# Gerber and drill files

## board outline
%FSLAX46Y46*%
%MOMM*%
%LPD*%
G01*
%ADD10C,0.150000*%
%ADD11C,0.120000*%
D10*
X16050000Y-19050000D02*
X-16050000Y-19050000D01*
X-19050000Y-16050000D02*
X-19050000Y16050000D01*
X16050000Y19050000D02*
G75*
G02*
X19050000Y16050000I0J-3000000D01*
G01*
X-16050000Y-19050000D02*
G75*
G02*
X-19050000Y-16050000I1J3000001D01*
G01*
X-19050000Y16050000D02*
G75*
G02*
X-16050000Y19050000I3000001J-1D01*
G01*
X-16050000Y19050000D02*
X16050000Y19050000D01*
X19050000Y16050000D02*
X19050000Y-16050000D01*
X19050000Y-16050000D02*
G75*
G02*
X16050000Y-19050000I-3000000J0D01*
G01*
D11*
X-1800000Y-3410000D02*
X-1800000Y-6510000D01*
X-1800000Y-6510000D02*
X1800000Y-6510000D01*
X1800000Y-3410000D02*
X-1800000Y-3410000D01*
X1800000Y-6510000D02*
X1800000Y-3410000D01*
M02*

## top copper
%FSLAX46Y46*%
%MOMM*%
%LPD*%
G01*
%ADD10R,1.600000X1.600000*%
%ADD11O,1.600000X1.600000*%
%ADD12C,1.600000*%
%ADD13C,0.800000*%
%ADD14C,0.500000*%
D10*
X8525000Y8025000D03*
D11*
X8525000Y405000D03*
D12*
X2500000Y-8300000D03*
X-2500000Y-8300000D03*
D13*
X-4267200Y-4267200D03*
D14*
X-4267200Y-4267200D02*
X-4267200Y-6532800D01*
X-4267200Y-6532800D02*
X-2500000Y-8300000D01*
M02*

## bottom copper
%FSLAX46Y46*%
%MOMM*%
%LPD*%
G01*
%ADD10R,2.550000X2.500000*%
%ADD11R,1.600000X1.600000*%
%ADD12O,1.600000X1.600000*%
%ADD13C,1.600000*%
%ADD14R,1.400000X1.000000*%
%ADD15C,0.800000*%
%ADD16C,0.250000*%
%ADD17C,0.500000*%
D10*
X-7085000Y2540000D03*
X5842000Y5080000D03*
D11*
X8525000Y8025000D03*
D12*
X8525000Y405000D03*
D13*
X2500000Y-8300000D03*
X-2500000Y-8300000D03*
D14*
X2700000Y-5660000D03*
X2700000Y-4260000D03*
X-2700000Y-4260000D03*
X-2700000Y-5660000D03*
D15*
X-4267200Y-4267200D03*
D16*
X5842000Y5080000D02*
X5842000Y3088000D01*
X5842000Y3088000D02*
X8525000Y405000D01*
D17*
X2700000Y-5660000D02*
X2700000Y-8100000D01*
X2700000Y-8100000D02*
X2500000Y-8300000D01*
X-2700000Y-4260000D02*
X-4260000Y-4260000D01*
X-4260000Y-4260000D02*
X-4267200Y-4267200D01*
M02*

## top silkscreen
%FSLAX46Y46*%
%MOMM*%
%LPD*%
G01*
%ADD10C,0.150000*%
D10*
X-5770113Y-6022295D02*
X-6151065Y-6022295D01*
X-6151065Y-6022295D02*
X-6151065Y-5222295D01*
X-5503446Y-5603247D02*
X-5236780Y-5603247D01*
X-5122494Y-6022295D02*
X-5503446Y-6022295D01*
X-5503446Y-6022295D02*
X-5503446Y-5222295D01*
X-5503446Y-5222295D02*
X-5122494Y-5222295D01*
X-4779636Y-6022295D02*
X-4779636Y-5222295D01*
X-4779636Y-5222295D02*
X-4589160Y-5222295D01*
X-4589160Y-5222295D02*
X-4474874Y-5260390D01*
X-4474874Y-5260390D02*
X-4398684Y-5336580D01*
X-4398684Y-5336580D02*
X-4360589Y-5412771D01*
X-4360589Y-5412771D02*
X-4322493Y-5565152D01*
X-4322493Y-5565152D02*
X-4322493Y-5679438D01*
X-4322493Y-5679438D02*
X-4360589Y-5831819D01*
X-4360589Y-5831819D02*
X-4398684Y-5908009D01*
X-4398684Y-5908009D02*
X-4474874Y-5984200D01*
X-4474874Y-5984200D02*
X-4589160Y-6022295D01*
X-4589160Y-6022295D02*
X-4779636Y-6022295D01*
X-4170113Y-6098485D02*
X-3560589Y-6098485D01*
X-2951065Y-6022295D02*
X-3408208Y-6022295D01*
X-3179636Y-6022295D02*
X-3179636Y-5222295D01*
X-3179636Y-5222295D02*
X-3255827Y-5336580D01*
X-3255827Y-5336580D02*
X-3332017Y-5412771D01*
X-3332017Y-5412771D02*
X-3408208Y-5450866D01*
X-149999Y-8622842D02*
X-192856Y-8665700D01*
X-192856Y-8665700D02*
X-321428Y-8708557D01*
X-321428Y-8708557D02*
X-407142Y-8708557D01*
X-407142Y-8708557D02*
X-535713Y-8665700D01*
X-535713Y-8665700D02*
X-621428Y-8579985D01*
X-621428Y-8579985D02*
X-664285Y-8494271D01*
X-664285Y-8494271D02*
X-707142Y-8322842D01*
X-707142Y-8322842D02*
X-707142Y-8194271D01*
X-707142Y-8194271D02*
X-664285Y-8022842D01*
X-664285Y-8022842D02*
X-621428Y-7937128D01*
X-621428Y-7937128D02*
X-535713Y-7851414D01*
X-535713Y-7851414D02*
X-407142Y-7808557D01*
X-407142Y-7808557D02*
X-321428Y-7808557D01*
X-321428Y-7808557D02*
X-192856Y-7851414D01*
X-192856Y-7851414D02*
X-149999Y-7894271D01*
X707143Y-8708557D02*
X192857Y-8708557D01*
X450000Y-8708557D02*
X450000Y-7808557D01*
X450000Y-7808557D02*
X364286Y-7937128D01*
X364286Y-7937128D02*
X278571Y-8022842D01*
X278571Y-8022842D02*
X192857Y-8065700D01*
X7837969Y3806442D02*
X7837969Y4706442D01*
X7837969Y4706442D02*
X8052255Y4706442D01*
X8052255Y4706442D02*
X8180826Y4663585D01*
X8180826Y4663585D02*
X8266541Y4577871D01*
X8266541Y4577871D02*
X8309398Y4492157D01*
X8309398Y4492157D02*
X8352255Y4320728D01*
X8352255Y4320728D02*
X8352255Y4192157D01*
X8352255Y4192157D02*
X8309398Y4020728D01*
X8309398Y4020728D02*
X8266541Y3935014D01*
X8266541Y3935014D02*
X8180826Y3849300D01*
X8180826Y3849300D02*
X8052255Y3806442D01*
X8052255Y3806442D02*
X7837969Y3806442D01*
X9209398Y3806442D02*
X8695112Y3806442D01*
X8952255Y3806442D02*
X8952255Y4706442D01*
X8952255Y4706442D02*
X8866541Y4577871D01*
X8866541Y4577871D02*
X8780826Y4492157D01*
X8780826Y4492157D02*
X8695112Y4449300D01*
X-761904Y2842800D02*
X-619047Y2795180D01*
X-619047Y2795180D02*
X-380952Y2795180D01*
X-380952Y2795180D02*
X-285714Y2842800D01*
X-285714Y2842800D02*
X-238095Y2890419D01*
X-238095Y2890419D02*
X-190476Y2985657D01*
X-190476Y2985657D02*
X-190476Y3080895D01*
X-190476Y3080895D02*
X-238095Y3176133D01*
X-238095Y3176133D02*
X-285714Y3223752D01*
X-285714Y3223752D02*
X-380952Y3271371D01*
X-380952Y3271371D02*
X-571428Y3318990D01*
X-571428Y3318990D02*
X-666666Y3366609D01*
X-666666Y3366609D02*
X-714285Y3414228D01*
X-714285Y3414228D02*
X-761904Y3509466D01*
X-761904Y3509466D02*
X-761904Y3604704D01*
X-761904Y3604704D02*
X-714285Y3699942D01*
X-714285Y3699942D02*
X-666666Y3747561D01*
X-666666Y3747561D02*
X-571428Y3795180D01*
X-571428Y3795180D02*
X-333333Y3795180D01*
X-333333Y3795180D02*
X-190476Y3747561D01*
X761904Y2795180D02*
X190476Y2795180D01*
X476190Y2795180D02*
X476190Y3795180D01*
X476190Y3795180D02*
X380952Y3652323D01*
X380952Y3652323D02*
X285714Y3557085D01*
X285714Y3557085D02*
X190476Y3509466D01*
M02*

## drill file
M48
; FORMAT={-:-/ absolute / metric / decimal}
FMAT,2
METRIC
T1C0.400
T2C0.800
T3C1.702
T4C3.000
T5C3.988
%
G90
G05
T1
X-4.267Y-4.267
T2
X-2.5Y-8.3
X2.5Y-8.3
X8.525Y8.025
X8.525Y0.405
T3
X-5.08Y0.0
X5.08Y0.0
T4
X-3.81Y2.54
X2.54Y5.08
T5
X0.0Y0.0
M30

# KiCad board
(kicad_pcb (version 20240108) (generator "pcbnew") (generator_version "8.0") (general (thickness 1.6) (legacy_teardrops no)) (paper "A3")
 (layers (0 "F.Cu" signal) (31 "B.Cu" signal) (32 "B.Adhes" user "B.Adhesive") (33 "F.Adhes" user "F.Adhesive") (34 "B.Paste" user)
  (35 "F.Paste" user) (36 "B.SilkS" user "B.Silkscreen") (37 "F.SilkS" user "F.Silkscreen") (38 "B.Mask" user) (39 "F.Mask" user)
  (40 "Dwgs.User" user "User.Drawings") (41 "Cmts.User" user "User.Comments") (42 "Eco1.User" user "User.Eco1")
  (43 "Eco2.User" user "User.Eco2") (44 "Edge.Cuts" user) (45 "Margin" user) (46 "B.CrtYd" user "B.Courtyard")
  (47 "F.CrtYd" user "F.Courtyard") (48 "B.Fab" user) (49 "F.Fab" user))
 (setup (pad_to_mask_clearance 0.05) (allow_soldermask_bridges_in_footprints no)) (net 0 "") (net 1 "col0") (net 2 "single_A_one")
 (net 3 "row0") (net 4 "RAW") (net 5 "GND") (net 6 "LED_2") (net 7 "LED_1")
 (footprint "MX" (layer "F.Cu") (at 0 0)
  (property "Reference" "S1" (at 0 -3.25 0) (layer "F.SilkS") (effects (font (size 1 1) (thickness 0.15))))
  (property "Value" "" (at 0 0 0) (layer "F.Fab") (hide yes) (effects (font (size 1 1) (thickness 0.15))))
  (pad "" np_thru_hole circle (at -5.08 0) (size 1.7018 1.7018) (drill 1.7018) (layers "*.Cu" "*.Mask"))
  (pad "" np_thru_hole circle (at -3.81 -2.54) (size 3 3) (drill 3) (layers "*.Cu" "*.Mask"))
  (pad "" np_thru_hole circle (at 0 0) (size 3.9878 3.9878) (drill 3.9878) (layers "*.Cu" "*.Mask"))
  (pad "" np_thru_hole circle (at 2.54 -5.08) (size 3 3) (drill 3) (layers "*.Cu" "*.Mask"))
  (pad "" np_thru_hole circle (at 5.08 0) (size 1.7018 1.7018) (drill 1.7018) (layers "*.Cu" "*.Mask"))
  (pad "1" smd rect (at -7.085 -2.54) (size 2.55 2.5) (layers "B.Cu" "B.Paste" "B.Mask") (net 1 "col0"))
  (pad "2" smd rect (at 5.842 -5.08) (size 2.55 2.5) (layers "B.Cu" "B.Paste" "B.Mask") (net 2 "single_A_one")))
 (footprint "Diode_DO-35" (layer "B.Cu") (at 8.525 -8.025 -90)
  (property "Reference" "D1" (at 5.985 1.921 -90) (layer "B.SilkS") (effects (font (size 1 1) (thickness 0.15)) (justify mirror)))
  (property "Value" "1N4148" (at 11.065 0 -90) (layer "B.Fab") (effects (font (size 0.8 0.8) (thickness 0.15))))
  (pad "1" thru_hole rect (at 0 0 270) (size 1.6 1.6) (drill 0.8) (layers "*.Cu" "*.Mask") (remove_unused_layers no) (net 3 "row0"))
  (pad "2" thru_hole oval (at 7.62 0 270) (size 1.6 1.6) (drill 0.8) (layers "*.Cu" "*.Mask") (remove_unused_layers no)
   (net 2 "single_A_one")))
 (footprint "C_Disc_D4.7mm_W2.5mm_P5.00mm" (layer "B.Cu") (at 2.5 8.3 180)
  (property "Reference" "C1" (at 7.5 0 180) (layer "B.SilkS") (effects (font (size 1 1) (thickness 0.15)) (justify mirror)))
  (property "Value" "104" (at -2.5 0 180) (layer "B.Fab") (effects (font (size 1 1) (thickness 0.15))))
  (pad "1" thru_hole circle (at 0 0) (size 1.6 1.6) (drill 0.8) (layers "*.Cu" "*.Mask") (remove_unused_layers no) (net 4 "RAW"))
  (pad "2" thru_hole circle (at 5 0) (size 1.6 1.6) (drill 0.8) (layers "*.Cu" "*.Mask") (remove_unused_layers no) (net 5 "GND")))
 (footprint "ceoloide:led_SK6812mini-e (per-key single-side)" (layer "B.Cu") (at 0 4.96)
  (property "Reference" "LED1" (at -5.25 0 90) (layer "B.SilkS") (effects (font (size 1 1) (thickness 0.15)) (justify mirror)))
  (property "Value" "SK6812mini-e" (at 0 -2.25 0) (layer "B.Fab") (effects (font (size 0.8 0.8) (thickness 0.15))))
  (fp_line (start -1.8 -1.55) (end -1.8 1.55) (stroke (width 0.12) (type solid)) (layer "Edge.Cuts"))
  (fp_line (start -1.8 1.55) (end 1.8 1.55) (stroke (width 0.12) (type solid)) (layer "Edge.Cuts"))
  (fp_line (start 1.8 -1.55) (end -1.8 -1.55) (stroke (width 0.12) (type solid)) (layer "Edge.Cuts"))
  (fp_line (start 1.8 1.55) (end 1.8 -1.55) (stroke (width 0.12) (type solid)) (layer "Edge.Cuts"))
  (pad "1" smd rect (at 2.7 0.7) (size 1.4 1) (layers "B.Cu" "B.Paste" "B.Mask") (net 4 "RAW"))
  (pad "2" smd rect (at 2.7 -0.7) (size 1.4 1) (layers "B.Cu" "B.Paste" "B.Mask") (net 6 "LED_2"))
  (pad "3" smd rect (at -2.7 -0.7) (size 1.4 1) (layers "B.Cu" "B.Paste" "B.Mask") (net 5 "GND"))
  (pad "4" smd rect (at -2.7 0.7) (size 1.4 1) (layers "B.Cu" "B.Paste" "B.Mask") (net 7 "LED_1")))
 (gr_line (start 16.05 19.05) (end -16.05 19.05) (stroke (width 0.15) (type solid)) (layer "Edge.Cuts"))
 (gr_line (start -19.05 16.05) (end -19.05 -16.05) (stroke (width 0.15) (type solid)) (layer "Edge.Cuts"))
 (gr_arc (start 16.05 -19.05) (mid 18.17132 -18.17132) (end 19.05 -16.05) (stroke (width 0.15) (type solid)) (layer "Edge.Cuts"))
 (gr_arc (start -16.05 19.05) (mid -18.17132 18.17132) (end -19.05 16.05) (stroke (width 0.15) (type solid)) (layer "Edge.Cuts"))
 (gr_arc (start -19.05 -16.05) (mid -18.17132 -18.17132) (end -16.05 -19.05) (stroke (width 0.15) (type solid)) (layer "Edge.Cuts"))
 (gr_line (start -16.05 -19.05) (end 16.05 -19.05) (stroke (width 0.15) (type solid)) (layer "Edge.Cuts"))
 (gr_line (start 19.05 -16.05) (end 19.05 16.05) (stroke (width 0.15) (type solid)) (layer "Edge.Cuts"))
 (gr_arc (start 19.05 16.05) (mid 18.17132 18.17132) (end 16.05 19.05) (stroke (width 0.15) (type solid)) (layer "Edge.Cuts"))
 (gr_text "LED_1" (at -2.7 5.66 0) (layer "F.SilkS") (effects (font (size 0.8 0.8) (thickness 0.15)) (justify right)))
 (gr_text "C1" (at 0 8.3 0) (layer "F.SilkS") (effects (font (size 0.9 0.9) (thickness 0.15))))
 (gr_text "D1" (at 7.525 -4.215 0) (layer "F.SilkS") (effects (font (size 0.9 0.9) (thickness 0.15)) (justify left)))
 (segment (start 5.842 -5.08) (end 5.842 -3.088) (width 0.25) (layer "B.Cu") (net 2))
 (segment (start 5.842 -3.088) (end 8.525 -0.405) (width 0.25) (layer "B.Cu") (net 2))
 (segment (start 2.7 5.66) (end 2.7 8.1) (width 0.5) (layer "B.Cu") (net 4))
 (segment (start 2.7 8.1) (end 2.5 8.3) (width 0.5) (layer "B.Cu") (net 4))
 (segment (start -4.2672 4.2672) (end -4.2672 6.5328) (width 0.5) (layer "F.Cu") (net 5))
 (segment (start -4.2672 6.5328) (end -2.5 8.3) (width 0.5) (layer "F.Cu") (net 5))
 (via (at -4.2672 4.2672) (size 0.8) (drill 0.4) (layers "F.Cu" "B.Cu") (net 5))
 (segment (start -2.7 4.26) (end -4.26 4.26) (width 0.5) (layer "B.Cu") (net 5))
 (segment (start -4.26 4.26) (end -4.2672 4.2672) (width 0.5) (layer "B.Cu") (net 5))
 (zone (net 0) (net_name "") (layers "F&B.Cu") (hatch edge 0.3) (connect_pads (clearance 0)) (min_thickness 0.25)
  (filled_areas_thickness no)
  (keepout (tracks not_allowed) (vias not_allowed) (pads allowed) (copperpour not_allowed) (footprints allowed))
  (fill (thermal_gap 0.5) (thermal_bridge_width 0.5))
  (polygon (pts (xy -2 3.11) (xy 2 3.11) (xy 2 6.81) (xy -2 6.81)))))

